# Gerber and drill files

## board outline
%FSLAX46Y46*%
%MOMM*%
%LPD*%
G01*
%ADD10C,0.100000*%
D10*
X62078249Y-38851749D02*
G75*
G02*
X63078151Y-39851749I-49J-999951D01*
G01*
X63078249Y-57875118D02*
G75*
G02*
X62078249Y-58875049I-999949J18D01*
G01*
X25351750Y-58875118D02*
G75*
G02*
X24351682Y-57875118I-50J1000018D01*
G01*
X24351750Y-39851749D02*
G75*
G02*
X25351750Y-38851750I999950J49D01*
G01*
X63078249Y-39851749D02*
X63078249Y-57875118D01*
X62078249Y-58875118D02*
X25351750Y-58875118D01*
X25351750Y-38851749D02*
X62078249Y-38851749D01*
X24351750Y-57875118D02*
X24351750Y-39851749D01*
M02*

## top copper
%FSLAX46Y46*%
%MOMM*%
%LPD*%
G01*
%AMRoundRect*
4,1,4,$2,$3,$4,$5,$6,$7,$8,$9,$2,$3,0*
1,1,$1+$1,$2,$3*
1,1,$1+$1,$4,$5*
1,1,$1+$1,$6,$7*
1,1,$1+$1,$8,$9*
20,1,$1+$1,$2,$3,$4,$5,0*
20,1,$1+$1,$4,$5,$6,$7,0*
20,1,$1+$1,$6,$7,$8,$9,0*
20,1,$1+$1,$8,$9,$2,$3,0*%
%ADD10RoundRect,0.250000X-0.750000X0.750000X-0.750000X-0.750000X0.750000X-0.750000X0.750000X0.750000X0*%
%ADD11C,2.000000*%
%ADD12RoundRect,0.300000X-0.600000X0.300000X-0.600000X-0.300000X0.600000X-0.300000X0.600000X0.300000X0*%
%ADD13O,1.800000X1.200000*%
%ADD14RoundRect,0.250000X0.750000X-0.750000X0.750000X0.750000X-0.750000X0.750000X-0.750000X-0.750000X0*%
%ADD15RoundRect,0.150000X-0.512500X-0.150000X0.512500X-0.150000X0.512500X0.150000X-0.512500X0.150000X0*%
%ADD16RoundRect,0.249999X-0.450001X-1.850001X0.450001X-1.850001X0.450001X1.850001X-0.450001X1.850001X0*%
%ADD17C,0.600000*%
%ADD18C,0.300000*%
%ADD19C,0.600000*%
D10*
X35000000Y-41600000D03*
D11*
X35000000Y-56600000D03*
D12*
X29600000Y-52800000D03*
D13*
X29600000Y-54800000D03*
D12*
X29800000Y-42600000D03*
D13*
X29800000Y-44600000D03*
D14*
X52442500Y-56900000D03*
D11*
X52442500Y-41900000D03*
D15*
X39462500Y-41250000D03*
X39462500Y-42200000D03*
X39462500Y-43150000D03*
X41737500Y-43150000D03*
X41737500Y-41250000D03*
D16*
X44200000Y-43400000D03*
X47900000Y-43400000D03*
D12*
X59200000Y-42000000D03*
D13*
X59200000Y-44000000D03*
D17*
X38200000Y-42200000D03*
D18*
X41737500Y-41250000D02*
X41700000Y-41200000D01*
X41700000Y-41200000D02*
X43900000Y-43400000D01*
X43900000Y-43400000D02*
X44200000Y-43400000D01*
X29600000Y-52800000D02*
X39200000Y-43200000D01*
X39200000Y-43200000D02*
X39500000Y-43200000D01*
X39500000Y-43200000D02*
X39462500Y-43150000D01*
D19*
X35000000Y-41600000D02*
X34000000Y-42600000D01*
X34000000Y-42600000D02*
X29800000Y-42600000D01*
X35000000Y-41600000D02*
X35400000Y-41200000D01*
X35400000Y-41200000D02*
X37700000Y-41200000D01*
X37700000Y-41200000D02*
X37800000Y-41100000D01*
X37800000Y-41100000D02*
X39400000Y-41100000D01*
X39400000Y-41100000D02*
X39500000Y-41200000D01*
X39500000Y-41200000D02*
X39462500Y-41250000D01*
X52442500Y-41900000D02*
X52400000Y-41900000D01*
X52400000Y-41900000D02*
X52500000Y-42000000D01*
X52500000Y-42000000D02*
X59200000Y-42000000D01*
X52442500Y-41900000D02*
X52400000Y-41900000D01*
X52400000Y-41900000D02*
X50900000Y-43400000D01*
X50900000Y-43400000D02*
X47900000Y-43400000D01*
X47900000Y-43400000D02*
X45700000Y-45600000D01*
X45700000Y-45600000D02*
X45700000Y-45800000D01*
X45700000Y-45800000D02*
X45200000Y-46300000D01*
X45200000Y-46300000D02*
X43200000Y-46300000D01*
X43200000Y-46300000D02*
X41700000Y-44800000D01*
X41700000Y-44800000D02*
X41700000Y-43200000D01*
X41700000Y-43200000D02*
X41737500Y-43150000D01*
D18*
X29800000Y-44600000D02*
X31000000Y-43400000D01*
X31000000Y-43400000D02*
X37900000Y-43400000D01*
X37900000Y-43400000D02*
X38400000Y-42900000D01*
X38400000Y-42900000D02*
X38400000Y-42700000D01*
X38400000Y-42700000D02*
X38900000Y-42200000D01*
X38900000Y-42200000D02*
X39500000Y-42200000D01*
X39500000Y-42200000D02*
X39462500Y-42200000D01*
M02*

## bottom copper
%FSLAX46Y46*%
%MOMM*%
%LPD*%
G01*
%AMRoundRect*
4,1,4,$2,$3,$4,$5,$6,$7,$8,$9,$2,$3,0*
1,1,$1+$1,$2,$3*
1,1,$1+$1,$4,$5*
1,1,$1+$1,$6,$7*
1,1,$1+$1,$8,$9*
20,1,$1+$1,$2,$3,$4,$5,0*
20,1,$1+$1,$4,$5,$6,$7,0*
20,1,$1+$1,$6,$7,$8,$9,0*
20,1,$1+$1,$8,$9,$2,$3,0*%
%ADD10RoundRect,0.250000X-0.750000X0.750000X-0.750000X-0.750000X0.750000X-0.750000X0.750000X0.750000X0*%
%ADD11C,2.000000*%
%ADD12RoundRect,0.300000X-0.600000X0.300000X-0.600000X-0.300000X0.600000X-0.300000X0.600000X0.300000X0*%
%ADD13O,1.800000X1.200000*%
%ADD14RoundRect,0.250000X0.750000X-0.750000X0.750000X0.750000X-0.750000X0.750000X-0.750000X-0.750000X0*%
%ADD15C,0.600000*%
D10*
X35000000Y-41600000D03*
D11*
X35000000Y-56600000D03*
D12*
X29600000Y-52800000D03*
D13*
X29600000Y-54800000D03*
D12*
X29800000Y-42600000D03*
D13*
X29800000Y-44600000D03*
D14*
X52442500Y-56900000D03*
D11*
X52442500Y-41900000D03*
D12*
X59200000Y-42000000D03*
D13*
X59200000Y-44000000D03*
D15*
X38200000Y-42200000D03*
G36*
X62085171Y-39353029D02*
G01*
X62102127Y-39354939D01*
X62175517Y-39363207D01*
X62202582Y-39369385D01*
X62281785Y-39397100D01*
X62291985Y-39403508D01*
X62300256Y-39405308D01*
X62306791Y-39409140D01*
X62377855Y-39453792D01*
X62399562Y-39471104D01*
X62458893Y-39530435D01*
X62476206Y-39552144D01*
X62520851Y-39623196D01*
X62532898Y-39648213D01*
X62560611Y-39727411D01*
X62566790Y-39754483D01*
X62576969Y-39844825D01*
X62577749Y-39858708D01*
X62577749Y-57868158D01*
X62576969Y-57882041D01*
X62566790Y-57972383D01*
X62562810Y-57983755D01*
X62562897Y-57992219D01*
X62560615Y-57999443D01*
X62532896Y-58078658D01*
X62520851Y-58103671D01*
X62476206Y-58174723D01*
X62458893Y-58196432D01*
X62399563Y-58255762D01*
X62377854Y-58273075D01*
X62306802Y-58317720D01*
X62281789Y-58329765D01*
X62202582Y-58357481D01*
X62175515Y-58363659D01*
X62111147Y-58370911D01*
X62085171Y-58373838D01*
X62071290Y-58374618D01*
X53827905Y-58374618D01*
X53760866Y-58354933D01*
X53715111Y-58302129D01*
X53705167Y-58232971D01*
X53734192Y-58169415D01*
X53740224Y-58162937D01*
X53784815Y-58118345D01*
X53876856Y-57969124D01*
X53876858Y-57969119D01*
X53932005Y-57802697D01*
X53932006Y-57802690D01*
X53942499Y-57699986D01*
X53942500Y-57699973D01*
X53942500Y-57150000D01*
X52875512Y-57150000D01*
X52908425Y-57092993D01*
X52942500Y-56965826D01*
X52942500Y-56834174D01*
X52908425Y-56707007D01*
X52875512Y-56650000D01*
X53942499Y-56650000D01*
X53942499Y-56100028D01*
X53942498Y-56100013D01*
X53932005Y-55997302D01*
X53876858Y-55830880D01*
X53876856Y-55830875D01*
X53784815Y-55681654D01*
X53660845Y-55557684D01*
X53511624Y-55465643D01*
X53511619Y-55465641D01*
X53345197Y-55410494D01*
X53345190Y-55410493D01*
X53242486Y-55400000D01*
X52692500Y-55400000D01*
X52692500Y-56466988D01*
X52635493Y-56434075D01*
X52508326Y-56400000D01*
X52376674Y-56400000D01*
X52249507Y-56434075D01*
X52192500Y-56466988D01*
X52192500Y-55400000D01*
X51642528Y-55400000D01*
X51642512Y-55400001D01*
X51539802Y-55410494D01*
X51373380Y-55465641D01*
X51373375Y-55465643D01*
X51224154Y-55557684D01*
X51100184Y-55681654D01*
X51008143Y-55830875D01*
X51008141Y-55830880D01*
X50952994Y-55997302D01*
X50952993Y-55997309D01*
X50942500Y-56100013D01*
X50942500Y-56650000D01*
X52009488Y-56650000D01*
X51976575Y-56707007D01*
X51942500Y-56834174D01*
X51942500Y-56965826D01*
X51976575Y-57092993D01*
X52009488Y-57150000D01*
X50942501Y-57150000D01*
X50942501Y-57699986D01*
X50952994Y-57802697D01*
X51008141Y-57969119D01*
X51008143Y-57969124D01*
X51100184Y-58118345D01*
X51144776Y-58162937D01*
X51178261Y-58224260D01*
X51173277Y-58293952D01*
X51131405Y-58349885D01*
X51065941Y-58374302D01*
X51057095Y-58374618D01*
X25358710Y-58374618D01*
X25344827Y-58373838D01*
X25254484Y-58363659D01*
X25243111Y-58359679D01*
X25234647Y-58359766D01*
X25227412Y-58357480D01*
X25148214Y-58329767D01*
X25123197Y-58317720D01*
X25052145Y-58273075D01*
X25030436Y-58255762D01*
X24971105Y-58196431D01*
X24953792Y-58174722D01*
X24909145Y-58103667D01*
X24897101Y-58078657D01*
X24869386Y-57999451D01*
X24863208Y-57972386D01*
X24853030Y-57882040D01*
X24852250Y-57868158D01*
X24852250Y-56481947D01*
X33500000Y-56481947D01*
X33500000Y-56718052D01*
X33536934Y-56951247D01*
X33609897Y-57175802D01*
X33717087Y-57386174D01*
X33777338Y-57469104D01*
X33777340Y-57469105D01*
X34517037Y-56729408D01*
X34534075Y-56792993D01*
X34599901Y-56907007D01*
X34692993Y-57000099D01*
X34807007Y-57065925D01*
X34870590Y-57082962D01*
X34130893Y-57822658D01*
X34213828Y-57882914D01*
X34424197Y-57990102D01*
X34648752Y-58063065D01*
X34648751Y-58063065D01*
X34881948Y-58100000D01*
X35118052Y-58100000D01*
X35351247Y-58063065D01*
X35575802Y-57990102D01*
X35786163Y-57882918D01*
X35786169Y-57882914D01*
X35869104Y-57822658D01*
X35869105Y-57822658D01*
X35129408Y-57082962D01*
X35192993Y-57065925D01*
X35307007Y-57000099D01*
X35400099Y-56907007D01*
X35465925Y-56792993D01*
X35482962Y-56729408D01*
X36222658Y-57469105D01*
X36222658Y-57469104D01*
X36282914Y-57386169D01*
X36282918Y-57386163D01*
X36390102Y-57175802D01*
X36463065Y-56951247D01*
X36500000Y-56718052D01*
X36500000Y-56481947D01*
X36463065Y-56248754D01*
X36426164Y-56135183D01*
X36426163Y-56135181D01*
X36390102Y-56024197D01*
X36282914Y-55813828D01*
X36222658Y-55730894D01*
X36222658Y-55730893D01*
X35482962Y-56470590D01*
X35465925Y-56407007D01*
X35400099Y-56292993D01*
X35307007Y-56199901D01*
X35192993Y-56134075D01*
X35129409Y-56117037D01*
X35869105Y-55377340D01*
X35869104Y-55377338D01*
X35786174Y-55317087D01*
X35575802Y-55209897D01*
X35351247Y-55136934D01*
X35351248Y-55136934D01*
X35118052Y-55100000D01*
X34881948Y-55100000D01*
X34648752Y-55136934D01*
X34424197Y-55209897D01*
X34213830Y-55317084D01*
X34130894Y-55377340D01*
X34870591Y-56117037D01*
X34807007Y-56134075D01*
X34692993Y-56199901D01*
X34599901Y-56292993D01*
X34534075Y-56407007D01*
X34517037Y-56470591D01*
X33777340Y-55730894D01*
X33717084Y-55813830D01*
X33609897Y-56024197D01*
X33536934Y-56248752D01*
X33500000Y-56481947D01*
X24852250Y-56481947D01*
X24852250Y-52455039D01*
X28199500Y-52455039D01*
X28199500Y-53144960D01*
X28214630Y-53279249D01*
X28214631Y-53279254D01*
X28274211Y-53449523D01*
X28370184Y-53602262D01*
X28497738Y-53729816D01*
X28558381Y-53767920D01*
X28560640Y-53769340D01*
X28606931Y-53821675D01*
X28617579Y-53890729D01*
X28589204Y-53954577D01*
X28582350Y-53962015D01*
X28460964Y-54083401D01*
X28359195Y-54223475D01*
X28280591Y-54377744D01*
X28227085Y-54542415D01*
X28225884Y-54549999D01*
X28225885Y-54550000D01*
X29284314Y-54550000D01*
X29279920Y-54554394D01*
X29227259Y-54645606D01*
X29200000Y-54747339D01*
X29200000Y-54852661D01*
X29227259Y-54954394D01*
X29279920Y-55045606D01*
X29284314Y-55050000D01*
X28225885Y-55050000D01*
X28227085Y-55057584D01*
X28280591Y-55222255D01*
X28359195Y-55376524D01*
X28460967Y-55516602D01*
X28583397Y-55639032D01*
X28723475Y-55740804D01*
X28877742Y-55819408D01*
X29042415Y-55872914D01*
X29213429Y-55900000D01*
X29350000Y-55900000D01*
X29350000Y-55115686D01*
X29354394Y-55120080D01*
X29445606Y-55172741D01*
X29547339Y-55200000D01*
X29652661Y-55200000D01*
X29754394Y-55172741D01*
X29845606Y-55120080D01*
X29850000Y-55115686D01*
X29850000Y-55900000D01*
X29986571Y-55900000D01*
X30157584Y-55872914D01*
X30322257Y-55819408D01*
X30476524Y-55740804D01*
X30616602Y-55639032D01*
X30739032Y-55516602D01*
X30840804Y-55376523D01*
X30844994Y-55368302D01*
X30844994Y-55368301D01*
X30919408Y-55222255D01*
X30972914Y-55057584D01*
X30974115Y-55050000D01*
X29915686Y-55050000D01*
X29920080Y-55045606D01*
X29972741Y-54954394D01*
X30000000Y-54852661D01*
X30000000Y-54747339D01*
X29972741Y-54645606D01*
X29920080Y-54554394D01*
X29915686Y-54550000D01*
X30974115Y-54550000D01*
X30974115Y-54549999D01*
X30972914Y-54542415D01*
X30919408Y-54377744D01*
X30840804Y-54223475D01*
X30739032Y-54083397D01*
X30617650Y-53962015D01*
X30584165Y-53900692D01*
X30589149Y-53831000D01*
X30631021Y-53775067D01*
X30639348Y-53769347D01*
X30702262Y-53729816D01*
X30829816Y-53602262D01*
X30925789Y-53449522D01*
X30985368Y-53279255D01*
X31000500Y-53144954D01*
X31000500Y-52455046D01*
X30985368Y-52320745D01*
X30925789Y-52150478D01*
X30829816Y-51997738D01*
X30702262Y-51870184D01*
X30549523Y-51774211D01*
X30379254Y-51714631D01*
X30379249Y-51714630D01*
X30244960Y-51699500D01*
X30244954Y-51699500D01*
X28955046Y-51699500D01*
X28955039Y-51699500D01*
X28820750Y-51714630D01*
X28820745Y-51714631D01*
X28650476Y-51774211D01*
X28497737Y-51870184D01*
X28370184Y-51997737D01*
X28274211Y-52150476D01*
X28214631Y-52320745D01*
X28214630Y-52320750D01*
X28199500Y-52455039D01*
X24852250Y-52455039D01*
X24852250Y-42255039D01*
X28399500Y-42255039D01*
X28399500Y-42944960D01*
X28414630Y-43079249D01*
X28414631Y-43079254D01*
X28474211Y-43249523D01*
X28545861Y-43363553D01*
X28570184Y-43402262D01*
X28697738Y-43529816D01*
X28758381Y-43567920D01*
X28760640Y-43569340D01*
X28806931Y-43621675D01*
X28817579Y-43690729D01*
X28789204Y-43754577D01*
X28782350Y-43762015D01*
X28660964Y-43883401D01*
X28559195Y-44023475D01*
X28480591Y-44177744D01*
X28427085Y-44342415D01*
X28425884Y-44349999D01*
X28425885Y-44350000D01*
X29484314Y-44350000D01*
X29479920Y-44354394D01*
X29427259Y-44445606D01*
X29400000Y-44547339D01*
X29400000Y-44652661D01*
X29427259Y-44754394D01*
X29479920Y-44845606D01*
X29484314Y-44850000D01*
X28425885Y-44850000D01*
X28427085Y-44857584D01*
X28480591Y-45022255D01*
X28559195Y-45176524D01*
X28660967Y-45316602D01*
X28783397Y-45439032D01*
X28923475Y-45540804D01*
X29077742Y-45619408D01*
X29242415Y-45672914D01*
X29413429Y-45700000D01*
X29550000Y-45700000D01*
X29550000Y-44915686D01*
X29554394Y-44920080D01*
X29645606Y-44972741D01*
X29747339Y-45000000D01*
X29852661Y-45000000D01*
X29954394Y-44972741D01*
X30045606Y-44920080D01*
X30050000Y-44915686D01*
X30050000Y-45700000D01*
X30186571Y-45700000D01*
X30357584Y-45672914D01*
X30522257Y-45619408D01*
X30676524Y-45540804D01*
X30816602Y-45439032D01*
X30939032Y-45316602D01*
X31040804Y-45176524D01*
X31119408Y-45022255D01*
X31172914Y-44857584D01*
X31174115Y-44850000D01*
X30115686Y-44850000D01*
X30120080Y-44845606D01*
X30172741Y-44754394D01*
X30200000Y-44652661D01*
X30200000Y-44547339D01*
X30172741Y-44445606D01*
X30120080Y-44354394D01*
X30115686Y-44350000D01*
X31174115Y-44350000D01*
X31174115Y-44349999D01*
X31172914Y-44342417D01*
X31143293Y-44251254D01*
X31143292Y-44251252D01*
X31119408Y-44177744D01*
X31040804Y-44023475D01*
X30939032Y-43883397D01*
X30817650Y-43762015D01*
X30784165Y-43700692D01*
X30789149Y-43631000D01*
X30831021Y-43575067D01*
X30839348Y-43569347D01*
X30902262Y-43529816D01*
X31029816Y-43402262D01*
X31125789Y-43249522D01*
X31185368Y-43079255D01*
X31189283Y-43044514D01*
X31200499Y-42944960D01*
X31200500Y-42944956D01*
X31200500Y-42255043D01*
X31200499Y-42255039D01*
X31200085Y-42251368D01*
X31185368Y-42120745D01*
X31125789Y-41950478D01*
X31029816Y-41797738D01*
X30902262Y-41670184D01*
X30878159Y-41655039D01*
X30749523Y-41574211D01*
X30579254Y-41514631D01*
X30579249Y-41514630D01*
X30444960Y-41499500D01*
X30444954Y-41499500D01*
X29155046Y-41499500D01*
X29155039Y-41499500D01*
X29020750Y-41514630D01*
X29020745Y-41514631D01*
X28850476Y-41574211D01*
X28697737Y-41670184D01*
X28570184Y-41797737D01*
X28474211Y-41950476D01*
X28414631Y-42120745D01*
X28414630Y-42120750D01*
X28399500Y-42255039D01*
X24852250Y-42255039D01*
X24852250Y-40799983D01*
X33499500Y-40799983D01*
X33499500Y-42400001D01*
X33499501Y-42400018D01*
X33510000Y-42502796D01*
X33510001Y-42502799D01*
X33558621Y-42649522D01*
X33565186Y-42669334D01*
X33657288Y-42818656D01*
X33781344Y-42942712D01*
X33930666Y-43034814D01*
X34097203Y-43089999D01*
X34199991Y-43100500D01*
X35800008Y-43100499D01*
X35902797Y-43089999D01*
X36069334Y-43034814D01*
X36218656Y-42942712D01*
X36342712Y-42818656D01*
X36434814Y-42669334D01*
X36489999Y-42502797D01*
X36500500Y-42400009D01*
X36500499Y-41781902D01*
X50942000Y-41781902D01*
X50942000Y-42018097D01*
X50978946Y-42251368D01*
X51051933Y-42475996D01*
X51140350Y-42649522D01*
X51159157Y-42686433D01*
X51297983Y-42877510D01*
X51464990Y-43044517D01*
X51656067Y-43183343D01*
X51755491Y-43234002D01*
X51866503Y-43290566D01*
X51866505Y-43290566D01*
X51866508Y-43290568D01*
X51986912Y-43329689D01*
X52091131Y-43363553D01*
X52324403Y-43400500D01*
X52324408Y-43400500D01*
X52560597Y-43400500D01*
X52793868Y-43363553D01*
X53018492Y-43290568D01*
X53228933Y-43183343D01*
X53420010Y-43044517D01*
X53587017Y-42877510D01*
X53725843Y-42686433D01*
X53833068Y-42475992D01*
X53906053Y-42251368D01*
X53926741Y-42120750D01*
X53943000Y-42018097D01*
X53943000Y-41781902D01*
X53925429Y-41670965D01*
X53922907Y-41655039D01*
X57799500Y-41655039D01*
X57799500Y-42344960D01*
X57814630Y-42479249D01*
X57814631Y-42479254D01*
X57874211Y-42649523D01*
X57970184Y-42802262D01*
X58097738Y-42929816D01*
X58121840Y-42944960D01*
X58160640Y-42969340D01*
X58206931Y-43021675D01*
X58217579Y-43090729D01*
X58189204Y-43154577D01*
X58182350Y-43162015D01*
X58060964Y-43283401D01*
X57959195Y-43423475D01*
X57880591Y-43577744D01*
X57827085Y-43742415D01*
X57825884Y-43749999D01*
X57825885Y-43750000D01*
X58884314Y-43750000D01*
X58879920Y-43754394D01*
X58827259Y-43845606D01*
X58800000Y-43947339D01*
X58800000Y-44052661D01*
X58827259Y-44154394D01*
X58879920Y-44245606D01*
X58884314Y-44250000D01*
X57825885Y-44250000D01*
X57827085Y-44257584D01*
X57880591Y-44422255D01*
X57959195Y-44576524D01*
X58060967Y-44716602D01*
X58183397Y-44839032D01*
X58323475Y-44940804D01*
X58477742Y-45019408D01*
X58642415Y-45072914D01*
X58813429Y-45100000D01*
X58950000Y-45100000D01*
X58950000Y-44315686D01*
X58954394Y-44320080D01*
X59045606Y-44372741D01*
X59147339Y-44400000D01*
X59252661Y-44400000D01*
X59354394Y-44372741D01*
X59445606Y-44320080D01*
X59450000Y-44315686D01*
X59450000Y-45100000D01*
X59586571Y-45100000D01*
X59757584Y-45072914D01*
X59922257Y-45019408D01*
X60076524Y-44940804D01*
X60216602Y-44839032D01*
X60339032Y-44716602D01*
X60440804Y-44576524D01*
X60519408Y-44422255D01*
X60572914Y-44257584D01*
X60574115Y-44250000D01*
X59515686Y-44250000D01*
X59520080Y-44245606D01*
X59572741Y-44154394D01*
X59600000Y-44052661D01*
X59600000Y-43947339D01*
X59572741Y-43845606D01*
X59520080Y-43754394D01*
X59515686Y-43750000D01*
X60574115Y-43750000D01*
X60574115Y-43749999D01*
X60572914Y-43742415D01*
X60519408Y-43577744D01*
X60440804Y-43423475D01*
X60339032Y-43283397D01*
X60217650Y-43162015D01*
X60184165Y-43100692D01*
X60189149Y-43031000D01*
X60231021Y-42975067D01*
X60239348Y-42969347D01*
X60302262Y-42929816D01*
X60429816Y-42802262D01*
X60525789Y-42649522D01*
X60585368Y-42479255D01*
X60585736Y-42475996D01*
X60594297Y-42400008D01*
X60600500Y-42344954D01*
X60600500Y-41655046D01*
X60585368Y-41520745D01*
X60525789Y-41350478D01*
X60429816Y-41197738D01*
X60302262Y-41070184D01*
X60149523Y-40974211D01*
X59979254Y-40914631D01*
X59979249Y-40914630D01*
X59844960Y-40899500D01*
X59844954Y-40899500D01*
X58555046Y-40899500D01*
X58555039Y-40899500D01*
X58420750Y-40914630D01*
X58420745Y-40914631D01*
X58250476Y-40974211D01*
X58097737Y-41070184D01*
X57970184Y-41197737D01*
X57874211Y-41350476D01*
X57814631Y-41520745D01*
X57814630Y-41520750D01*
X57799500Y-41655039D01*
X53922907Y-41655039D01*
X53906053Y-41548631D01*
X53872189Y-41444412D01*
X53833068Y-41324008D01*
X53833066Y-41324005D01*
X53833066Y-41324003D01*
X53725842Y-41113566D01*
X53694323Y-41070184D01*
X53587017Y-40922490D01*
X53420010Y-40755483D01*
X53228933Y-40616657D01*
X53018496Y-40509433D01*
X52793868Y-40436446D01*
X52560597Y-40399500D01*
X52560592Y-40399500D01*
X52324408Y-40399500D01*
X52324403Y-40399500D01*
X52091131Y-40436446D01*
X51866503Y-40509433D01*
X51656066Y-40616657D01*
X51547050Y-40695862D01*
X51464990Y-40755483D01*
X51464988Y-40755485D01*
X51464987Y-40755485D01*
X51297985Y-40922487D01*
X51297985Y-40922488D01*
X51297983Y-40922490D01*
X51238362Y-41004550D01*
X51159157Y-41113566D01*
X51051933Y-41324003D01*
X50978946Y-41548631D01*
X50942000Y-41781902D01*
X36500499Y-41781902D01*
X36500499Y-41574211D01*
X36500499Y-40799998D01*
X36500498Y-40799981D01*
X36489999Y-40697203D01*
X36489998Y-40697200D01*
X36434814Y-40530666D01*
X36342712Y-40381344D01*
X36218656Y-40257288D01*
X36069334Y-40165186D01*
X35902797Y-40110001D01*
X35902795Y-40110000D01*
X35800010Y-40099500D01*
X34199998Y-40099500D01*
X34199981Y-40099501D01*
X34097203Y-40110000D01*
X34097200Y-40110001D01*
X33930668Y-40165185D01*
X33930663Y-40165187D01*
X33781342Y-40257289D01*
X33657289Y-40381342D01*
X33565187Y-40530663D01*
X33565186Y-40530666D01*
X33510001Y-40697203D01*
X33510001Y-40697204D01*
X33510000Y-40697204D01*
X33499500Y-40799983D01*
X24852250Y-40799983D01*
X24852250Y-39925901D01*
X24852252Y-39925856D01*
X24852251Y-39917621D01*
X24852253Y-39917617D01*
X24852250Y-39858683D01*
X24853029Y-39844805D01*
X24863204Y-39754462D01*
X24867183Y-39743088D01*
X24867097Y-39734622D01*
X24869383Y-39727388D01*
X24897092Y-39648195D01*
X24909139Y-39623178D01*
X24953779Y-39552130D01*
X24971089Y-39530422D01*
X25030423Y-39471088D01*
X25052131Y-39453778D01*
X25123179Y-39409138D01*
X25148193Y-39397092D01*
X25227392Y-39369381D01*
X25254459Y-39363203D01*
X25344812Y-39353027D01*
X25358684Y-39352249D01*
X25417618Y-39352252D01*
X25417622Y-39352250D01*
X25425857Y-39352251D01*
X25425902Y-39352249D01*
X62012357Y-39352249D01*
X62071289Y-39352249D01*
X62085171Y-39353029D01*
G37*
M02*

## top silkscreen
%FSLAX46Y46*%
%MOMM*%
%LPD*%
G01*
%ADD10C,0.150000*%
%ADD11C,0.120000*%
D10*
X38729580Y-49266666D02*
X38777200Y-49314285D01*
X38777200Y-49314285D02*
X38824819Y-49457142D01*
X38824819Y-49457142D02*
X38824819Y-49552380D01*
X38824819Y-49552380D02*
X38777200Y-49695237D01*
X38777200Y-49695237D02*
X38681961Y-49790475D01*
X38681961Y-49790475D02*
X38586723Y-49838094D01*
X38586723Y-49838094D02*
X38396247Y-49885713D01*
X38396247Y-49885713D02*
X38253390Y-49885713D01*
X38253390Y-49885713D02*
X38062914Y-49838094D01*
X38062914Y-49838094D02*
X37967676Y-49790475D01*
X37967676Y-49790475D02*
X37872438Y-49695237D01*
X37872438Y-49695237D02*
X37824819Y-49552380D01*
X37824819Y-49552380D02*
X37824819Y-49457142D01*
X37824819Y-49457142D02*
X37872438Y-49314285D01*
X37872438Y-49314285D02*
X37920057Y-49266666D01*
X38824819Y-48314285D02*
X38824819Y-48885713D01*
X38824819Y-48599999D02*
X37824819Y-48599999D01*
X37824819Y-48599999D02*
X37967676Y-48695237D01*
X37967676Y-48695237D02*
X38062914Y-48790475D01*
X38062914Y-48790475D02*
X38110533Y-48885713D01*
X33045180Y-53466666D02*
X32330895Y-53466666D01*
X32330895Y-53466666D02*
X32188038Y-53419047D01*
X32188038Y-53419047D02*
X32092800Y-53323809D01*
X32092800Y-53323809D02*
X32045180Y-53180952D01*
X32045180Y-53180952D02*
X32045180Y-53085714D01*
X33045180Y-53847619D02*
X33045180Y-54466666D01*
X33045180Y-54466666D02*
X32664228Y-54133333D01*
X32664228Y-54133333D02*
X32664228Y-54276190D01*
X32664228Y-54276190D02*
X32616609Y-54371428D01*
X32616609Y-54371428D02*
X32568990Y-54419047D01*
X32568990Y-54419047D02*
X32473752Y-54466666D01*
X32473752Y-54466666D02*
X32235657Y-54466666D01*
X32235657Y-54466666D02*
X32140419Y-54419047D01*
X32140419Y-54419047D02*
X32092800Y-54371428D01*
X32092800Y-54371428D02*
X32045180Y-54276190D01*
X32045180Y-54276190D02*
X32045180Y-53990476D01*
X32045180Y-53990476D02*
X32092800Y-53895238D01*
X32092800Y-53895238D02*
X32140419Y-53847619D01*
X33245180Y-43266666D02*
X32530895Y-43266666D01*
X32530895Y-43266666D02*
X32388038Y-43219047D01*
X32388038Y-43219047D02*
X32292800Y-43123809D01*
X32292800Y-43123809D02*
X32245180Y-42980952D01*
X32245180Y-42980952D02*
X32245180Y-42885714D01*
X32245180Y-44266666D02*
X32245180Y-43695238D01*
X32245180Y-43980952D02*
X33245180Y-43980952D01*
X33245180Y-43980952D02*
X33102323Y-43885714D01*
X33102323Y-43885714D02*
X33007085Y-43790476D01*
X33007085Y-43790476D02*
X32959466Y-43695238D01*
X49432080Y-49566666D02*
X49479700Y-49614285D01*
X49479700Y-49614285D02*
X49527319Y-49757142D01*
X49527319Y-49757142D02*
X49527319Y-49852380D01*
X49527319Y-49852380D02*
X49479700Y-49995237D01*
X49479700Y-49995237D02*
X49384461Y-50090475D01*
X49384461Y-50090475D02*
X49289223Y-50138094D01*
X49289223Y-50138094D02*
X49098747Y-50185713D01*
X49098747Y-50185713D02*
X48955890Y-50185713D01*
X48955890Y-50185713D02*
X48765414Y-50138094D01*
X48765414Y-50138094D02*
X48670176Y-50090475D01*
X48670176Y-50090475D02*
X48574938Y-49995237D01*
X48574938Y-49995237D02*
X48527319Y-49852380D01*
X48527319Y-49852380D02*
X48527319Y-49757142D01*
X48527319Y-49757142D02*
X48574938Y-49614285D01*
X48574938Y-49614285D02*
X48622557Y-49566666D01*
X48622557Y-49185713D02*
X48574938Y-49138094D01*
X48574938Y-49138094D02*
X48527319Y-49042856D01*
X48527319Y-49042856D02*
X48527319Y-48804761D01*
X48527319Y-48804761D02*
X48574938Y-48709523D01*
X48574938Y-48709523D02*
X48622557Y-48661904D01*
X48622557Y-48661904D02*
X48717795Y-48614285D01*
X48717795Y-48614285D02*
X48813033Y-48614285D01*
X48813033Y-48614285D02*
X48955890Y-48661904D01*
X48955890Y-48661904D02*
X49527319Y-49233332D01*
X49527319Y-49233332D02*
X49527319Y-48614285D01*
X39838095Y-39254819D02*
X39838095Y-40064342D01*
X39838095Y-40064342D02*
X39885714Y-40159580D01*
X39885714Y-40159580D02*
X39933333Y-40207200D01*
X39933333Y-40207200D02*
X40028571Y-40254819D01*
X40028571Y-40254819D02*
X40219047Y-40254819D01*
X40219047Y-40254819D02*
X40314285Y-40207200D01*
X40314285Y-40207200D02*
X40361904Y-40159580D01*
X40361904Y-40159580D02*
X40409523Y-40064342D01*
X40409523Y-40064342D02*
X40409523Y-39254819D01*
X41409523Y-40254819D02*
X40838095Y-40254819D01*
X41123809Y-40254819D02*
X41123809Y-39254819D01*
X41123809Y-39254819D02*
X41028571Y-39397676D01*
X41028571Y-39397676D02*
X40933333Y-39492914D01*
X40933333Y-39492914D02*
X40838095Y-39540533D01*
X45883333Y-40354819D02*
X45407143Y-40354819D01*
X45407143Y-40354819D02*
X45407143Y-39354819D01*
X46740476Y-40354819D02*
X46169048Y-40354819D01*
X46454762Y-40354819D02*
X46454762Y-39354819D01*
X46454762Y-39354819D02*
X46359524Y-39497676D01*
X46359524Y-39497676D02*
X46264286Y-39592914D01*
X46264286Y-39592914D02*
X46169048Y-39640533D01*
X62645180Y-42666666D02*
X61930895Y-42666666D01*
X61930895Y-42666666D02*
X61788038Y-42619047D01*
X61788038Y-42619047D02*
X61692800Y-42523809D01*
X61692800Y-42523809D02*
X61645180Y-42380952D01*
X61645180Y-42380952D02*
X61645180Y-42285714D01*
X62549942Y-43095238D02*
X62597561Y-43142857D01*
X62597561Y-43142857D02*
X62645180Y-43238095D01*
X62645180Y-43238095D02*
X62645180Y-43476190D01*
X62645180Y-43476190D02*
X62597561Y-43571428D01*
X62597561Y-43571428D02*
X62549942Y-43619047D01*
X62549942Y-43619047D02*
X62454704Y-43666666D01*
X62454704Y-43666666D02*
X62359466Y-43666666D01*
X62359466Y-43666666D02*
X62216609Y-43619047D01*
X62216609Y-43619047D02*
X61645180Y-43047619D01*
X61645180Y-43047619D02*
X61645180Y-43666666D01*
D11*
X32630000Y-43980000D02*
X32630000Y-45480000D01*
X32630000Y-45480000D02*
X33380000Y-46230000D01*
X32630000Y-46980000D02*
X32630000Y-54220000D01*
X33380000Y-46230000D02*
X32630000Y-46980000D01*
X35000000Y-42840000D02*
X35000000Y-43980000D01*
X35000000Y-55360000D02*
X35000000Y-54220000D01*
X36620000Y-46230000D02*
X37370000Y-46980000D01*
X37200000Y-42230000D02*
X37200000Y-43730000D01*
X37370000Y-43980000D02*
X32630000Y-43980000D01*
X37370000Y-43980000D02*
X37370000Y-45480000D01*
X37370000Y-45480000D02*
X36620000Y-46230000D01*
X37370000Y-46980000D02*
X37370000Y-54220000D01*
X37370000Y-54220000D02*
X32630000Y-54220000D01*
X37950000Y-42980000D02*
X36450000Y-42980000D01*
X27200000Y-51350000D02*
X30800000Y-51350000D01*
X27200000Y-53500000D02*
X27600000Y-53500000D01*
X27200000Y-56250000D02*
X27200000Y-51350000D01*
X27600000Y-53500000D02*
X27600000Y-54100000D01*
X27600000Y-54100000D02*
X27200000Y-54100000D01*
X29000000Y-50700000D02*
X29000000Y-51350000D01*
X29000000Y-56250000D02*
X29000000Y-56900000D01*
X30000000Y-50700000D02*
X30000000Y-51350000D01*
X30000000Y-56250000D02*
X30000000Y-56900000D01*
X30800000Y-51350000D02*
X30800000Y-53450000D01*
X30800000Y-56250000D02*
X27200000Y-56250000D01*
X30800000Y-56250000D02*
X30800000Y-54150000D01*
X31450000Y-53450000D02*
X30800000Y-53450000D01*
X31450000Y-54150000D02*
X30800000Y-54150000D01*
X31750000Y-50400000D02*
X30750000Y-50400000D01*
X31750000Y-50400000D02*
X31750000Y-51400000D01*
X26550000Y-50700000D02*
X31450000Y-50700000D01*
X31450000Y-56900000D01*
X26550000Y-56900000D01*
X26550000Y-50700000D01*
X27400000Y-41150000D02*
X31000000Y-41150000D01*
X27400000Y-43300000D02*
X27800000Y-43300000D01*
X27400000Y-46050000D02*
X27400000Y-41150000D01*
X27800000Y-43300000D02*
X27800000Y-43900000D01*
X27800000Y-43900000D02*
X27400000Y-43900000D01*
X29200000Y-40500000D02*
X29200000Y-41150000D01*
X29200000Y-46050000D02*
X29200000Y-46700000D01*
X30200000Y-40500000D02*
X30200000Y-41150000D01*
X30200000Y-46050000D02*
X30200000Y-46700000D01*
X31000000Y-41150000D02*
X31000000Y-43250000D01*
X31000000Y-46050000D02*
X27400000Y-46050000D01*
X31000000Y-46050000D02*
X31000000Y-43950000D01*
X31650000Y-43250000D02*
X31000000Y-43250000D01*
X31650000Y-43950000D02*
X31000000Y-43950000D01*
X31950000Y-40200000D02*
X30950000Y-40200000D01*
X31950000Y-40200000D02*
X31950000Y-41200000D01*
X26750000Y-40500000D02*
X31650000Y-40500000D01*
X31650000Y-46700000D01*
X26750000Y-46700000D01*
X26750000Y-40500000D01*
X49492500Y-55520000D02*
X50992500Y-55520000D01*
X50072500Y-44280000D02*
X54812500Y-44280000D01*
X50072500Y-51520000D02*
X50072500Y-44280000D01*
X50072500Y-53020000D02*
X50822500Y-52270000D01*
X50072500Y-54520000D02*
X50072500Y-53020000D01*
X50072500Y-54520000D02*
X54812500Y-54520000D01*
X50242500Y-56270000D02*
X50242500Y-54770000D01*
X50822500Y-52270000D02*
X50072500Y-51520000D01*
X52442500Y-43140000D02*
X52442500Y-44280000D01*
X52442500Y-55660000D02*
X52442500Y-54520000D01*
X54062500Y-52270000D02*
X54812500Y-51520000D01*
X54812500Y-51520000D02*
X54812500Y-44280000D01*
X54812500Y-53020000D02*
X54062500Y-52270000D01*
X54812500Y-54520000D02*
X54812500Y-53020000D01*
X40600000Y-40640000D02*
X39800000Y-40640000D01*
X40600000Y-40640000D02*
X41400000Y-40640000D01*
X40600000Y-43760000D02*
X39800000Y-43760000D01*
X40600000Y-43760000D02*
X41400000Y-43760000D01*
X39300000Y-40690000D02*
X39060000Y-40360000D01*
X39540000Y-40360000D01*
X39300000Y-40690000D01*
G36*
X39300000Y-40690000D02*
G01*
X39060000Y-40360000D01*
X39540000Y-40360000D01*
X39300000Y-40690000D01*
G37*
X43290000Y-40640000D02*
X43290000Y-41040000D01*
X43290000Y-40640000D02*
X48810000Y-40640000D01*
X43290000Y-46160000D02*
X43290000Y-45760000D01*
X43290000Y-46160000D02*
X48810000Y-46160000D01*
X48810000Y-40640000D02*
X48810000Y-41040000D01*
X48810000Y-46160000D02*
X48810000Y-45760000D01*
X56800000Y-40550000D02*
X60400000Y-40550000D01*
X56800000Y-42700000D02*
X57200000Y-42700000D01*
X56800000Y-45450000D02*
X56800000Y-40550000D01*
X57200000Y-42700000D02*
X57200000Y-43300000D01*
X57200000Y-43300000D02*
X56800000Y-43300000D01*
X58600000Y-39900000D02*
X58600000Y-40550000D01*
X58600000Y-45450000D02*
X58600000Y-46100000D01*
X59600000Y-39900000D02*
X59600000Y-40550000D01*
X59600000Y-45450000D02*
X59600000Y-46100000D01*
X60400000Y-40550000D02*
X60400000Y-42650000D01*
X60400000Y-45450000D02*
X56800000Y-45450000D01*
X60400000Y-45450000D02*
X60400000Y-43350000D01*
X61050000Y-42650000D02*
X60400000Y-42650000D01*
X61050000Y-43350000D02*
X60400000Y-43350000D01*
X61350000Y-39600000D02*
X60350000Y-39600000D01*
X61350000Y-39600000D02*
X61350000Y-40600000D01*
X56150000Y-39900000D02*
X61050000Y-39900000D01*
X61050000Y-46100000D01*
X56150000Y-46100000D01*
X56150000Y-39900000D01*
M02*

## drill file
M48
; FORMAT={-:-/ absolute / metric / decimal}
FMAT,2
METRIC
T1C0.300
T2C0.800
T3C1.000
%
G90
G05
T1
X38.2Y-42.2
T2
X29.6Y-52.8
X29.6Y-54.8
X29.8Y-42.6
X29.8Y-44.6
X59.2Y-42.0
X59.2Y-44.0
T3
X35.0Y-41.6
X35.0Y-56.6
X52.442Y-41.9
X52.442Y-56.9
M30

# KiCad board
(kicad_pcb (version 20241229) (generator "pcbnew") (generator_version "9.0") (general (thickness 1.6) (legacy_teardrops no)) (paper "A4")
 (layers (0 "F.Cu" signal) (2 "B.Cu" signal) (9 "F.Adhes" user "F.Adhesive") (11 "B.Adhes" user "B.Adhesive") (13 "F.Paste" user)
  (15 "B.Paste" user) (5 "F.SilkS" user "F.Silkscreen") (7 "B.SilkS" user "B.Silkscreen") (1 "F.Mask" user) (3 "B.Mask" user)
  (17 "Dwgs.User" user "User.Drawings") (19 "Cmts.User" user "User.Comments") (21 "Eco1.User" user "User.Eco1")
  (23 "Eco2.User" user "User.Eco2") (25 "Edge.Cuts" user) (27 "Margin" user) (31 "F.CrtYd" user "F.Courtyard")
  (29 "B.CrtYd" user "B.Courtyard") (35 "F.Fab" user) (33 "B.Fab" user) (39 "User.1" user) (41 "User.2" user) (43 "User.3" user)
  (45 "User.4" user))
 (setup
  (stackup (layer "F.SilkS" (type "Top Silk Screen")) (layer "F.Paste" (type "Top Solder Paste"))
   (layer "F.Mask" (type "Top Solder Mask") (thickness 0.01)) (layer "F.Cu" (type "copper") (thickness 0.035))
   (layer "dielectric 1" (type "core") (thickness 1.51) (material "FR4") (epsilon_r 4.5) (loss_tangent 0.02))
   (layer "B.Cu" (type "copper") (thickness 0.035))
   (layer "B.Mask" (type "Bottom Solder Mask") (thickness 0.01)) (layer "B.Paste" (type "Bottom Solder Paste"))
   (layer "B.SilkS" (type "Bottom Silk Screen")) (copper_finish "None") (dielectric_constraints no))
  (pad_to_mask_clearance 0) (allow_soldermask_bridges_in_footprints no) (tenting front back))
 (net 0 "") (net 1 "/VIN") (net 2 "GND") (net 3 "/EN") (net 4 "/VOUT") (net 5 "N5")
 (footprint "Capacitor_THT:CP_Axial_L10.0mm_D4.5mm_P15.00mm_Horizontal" (layer "F.Cu") (at 35 41.6 -90)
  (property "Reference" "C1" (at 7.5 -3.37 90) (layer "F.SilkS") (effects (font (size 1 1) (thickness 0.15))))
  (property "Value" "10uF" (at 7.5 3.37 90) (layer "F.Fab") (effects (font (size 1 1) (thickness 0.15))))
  (fp_line (start 2.38 2.37) (end 3.88 2.37) (stroke (width 0.12) (type solid)) (layer "F.SilkS"))
  (fp_line (start 3.88 2.37) (end 4.63 1.62) (stroke (width 0.12) (type solid)) (layer "F.SilkS"))
  (fp_line (start 5.38 2.37) (end 12.62 2.37) (stroke (width 0.12) (type solid)) (layer "F.SilkS"))
  (fp_line (start 4.63 1.62) (end 5.38 2.37) (stroke (width 0.12) (type solid)) (layer "F.SilkS"))
  (fp_line (start 1.24 0) (end 2.38 0) (stroke (width 0.12) (type solid)) (layer "F.SilkS"))
  (fp_line (start 13.76 0) (end 12.62 0) (stroke (width 0.12) (type solid)) (layer "F.SilkS"))
  (fp_line (start 4.63 -1.62) (end 5.38 -2.37) (stroke (width 0.12) (type solid)) (layer "F.SilkS"))
  (fp_line (start 0.63 -2.2) (end 2.13 -2.2) (stroke (width 0.12) (type solid)) (layer "F.SilkS"))
  (fp_line (start 2.38 -2.37) (end 2.38 2.37) (stroke (width 0.12) (type solid)) (layer "F.SilkS"))
  (fp_line (start 2.38 -2.37) (end 3.88 -2.37) (stroke (width 0.12) (type solid)) (layer "F.SilkS"))
  (fp_line (start 3.88 -2.37) (end 4.63 -1.62) (stroke (width 0.12) (type solid)) (layer "F.SilkS"))
  (fp_line (start 5.38 -2.37) (end 12.62 -2.37) (stroke (width 0.12) (type solid)) (layer "F.SilkS"))
  (fp_line (start 12.62 -2.37) (end 12.62 2.37) (stroke (width 0.12) (type solid)) (layer "F.SilkS"))
  (fp_line (start 1.38 -2.95) (end 1.38 -1.45) (stroke (width 0.12) (type solid)) (layer "F.SilkS"))
  (pad "1" thru_hole roundrect (at 0 0 270) (size 2 2) (drill 1) (layers "*.Cu" "*.Mask") (remove_unused_layers no) (roundrect_rratio 0.125)
   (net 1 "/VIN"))
  (pad "2" thru_hole circle (at 15 0 270) (size 2 2) (drill 1) (layers "*.Cu" "*.Mask") (remove_unused_layers no) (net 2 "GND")))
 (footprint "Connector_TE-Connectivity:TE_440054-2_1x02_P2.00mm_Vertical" (layer "F.Cu") (at 29.6 52.8 -90)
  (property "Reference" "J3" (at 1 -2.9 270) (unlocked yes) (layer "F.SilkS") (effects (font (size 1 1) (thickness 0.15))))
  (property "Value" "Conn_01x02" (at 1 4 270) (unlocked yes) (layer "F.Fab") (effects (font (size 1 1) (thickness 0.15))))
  (fp_line (start -1.45 2.4) (end -1.45 -1.2) (stroke (width 0.12) (type solid)) (layer "F.SilkS"))
  (fp_line (start 0.7 2.4) (end 0.7 2) (stroke (width 0.12) (type solid)) (layer "F.SilkS"))
  (fp_line (start 3.45 2.4) (end -1.45 2.4) (stroke (width 0.12) (type solid)) (layer "F.SilkS"))
  (fp_line (start 0.7 2) (end 1.3 2) (stroke (width 0.12) (type solid)) (layer "F.SilkS"))
  (fp_line (start 1.3 2) (end 1.3 2.4) (stroke (width 0.12) (type solid)) (layer "F.SilkS"))
  (fp_line (start -2.1 0.6) (end -1.45 0.6) (stroke (width 0.12) (type solid)) (layer "F.SilkS"))
  (fp_line (start 3.45 0.6) (end 4.1 0.6) (stroke (width 0.12) (type solid)) (layer "F.SilkS"))
  (fp_line (start -2.1 -0.4) (end -1.45 -0.4) (stroke (width 0.12) (type solid)) (layer "F.SilkS"))
  (fp_line (start 3.45 -0.4) (end 4.1 -0.4) (stroke (width 0.12) (type solid)) (layer "F.SilkS"))
  (fp_line (start -1.45 -1.2) (end 0.65 -1.2) (stroke (width 0.12) (type solid)) (layer "F.SilkS"))
  (fp_line (start 3.45 -1.2) (end 3.45 2.4) (stroke (width 0.12) (type solid)) (layer "F.SilkS"))
  (fp_line (start 3.45 -1.2) (end 1.35 -1.2) (stroke (width 0.12) (type solid)) (layer "F.SilkS"))
  (fp_line (start 0.65 -1.85) (end 0.65 -1.2) (stroke (width 0.12) (type solid)) (layer "F.SilkS"))
  (fp_line (start 1.35 -1.85) (end 1.35 -1.2) (stroke (width 0.12) (type solid)) (layer "F.SilkS"))
  (fp_line (start -2.4 -2.15) (end -2.4 -1.15) (stroke (width 0.12) (type solid)) (layer "F.SilkS"))
  (fp_line (start -2.4 -2.15) (end -1.4 -2.15) (stroke (width 0.12) (type solid)) (layer "F.SilkS"))
  (fp_rect (start -2.1 -1.85) (end 4.1 3.05) (stroke (width 0.12) (type solid)) (fill no) (layer "F.SilkS"))
  (pad "1" thru_hole roundrect (at 0 0 270) (size 1.2 1.8) (drill 0.8) (layers "*.Cu" "*.Mask") (remove_unused_layers no)
   (roundrect_rratio 0.25) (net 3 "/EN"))
  (pad "2" thru_hole oval (at 2 0 270) (size 1.2 1.8) (drill 0.8) (layers "*.Cu" "*.Mask") (remove_unused_layers no) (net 2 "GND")))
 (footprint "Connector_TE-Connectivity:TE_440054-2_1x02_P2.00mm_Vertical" (layer "F.Cu") (at 29.8 42.6 -90)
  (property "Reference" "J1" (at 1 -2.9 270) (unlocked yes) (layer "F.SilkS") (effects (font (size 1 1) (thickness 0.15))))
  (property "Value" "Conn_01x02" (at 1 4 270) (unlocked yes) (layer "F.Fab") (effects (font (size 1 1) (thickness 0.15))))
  (fp_line (start -1.45 2.4) (end -1.45 -1.2) (stroke (width 0.12) (type solid)) (layer "F.SilkS"))
  (fp_line (start 0.7 2.4) (end 0.7 2) (stroke (width 0.12) (type solid)) (layer "F.SilkS"))
  (fp_line (start 3.45 2.4) (end -1.45 2.4) (stroke (width 0.12) (type solid)) (layer "F.SilkS"))
  (fp_line (start 0.7 2) (end 1.3 2) (stroke (width 0.12) (type solid)) (layer "F.SilkS"))
  (fp_line (start 1.3 2) (end 1.3 2.4) (stroke (width 0.12) (type solid)) (layer "F.SilkS"))
  (fp_line (start -2.1 0.6) (end -1.45 0.6) (stroke (width 0.12) (type solid)) (layer "F.SilkS"))
  (fp_line (start 3.45 0.6) (end 4.1 0.6) (stroke (width 0.12) (type solid)) (layer "F.SilkS"))
  (fp_line (start -2.1 -0.4) (end -1.45 -0.4) (stroke (width 0.12) (type solid)) (layer "F.SilkS"))
  (fp_line (start 3.45 -0.4) (end 4.1 -0.4) (stroke (width 0.12) (type solid)) (layer "F.SilkS"))
  (fp_line (start -1.45 -1.2) (end 0.65 -1.2) (stroke (width 0.12) (type solid)) (layer "F.SilkS"))
  (fp_line (start 3.45 -1.2) (end 3.45 2.4) (stroke (width 0.12) (type solid)) (layer "F.SilkS"))
  (fp_line (start 3.45 -1.2) (end 1.35 -1.2) (stroke (width 0.12) (type solid)) (layer "F.SilkS"))
  (fp_line (start 0.65 -1.85) (end 0.65 -1.2) (stroke (width 0.12) (type solid)) (layer "F.SilkS"))
  (fp_line (start 1.35 -1.85) (end 1.35 -1.2) (stroke (width 0.12) (type solid)) (layer "F.SilkS"))
  (fp_line (start -2.4 -2.15) (end -2.4 -1.15) (stroke (width 0.12) (type solid)) (layer "F.SilkS"))
  (fp_line (start -2.4 -2.15) (end -1.4 -2.15) (stroke (width 0.12) (type solid)) (layer "F.SilkS"))
  (fp_rect (start -2.1 -1.85) (end 4.1 3.05) (stroke (width 0.12) (type solid)) (fill no) (layer "F.SilkS"))
  (pad "1" thru_hole roundrect (at 0 0 270) (size 1.2 1.8) (drill 0.8) (layers "*.Cu" "*.Mask") (remove_unused_layers no)
   (roundrect_rratio 0.25) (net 1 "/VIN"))
  (pad "2" thru_hole oval (at 2 0 270) (size 1.2 1.8) (drill 0.8) (layers "*.Cu" "*.Mask") (remove_unused_layers no) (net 2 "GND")))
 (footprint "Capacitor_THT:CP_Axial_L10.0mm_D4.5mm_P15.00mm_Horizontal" (layer "F.Cu") (at 52.4425 56.9 90)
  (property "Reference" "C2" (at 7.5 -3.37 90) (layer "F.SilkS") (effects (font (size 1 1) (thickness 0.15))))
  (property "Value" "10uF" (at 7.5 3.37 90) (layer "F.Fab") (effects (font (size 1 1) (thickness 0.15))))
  (fp_line (start 1.38 -2.95) (end 1.38 -1.45) (stroke (width 0.12) (type solid)) (layer "F.SilkS"))
  (fp_line (start 12.62 -2.37) (end 12.62 2.37) (stroke (width 0.12) (type solid)) (layer "F.SilkS"))
  (fp_line (start 5.38 -2.37) (end 12.62 -2.37) (stroke (width 0.12) (type solid)) (layer "F.SilkS"))
  (fp_line (start 3.88 -2.37) (end 4.63 -1.62) (stroke (width 0.12) (type solid)) (layer "F.SilkS"))
  (fp_line (start 2.38 -2.37) (end 3.88 -2.37) (stroke (width 0.12) (type solid)) (layer "F.SilkS"))
  (fp_line (start 2.38 -2.37) (end 2.38 2.37) (stroke (width 0.12) (type solid)) (layer "F.SilkS"))
  (fp_line (start 0.63 -2.2) (end 2.13 -2.2) (stroke (width 0.12) (type solid)) (layer "F.SilkS"))
  (fp_line (start 4.63 -1.62) (end 5.38 -2.37) (stroke (width 0.12) (type solid)) (layer "F.SilkS"))
  (fp_line (start 13.76 0) (end 12.62 0) (stroke (width 0.12) (type solid)) (layer "F.SilkS"))
  (fp_line (start 1.24 0) (end 2.38 0) (stroke (width 0.12) (type solid)) (layer "F.SilkS"))
  (fp_line (start 4.63 1.62) (end 5.38 2.37) (stroke (width 0.12) (type solid)) (layer "F.SilkS"))
  (fp_line (start 5.38 2.37) (end 12.62 2.37) (stroke (width 0.12) (type solid)) (layer "F.SilkS"))
  (fp_line (start 3.88 2.37) (end 4.63 1.62) (stroke (width 0.12) (type solid)) (layer "F.SilkS"))
  (fp_line (start 2.38 2.37) (end 3.88 2.37) (stroke (width 0.12) (type solid)) (layer "F.SilkS"))
  (pad "1" thru_hole roundrect (at 0 0 90) (size 2 2) (drill 1) (layers "*.Cu" "*.Mask") (remove_unused_layers no) (roundrect_rratio 0.125)
   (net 2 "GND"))
  (pad "2" thru_hole circle (at 15 0 90) (size 2 2) (drill 1) (layers "*.Cu" "*.Mask") (remove_unused_layers no) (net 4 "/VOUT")))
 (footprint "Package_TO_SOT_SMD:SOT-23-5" (layer "F.Cu") (at 40.6 42.2)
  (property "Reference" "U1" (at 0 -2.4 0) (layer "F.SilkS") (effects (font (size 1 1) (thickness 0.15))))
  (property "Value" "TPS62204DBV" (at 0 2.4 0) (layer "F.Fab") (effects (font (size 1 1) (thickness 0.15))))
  (fp_line (start 0 -1.56) (end -0.8 -1.56) (stroke (width 0.12) (type solid)) (layer "F.SilkS"))
  (fp_line (start 0 -1.56) (end 0.8 -1.56) (stroke (width 0.12) (type solid)) (layer "F.SilkS"))
  (fp_line (start 0 1.56) (end -0.8 1.56) (stroke (width 0.12) (type solid)) (layer "F.SilkS"))
  (fp_line (start 0 1.56) (end 0.8 1.56) (stroke (width 0.12) (type solid)) (layer "F.SilkS"))
  (fp_poly (pts (xy -1.3 -1.51) (xy -1.54 -1.84) (xy -1.06 -1.84)) (stroke (width 0.12) (type solid)) (fill yes) (layer "F.SilkS"))
  (pad "1" smd roundrect (at -1.1375 -0.95) (size 1.325 0.6) (layers "F.Cu" "F.Mask" "F.Paste") (roundrect_rratio 0.25) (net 1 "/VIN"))
  (pad "2" smd roundrect (at -1.1375 0) (size 1.325 0.6) (layers "F.Cu" "F.Mask" "F.Paste") (roundrect_rratio 0.25) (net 2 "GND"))
  (pad "3" smd roundrect (at -1.1375 0.95) (size 1.325 0.6) (layers "F.Cu" "F.Mask" "F.Paste") (roundrect_rratio 0.25) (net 3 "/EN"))
  (pad "4" smd roundrect (at 1.1375 0.95) (size 1.325 0.6) (layers "F.Cu" "F.Mask" "F.Paste") (roundrect_rratio 0.25) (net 4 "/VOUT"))
  (pad "5" smd roundrect (at 1.1375 -0.95) (size 1.325 0.6) (layers "F.Cu" "F.Mask" "F.Paste") (roundrect_rratio 0.25) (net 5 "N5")))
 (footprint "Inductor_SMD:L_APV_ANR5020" (layer "F.Cu") (at 46.05 43.4)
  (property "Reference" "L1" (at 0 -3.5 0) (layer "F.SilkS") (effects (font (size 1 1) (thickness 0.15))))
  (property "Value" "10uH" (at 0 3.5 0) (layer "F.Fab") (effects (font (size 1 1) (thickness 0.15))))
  (fp_line (start -2.76 -2.76) (end -2.76 -2.36) (stroke (width 0.12) (type solid)) (layer "F.SilkS"))
  (fp_line (start -2.76 -2.76) (end 2.76 -2.76) (stroke (width 0.12) (type solid)) (layer "F.SilkS"))
  (fp_line (start -2.76 2.76) (end -2.76 2.36) (stroke (width 0.12) (type solid)) (layer "F.SilkS"))
  (fp_line (start -2.76 2.76) (end 2.76 2.76) (stroke (width 0.12) (type solid)) (layer "F.SilkS"))
  (fp_line (start 2.76 -2.76) (end 2.76 -2.36) (stroke (width 0.12) (type solid)) (layer "F.SilkS"))
  (fp_line (start 2.76 2.76) (end 2.76 2.36) (stroke (width 0.12) (type solid)) (layer "F.SilkS"))
  (pad "1" smd roundrect (at -1.85 0) (size 1.4 4.2) (layers "F.Cu" "F.Mask" "F.Paste") (roundrect_rratio 0.178571) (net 5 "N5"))
  (pad "2" smd roundrect (at 1.85 0) (size 1.4 4.2) (layers "F.Cu" "F.Mask" "F.Paste") (roundrect_rratio 0.178571) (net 4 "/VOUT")))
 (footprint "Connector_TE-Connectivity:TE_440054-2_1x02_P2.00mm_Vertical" (layer "F.Cu") (at 59.2 42 -90)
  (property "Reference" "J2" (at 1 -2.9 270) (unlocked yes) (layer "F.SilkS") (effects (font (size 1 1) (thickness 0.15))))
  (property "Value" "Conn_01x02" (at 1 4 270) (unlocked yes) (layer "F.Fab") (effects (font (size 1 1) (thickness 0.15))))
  (fp_line (start -1.45 2.4) (end -1.45 -1.2) (stroke (width 0.12) (type solid)) (layer "F.SilkS"))
  (fp_line (start 0.7 2.4) (end 0.7 2) (stroke (width 0.12) (type solid)) (layer "F.SilkS"))
  (fp_line (start 3.45 2.4) (end -1.45 2.4) (stroke (width 0.12) (type solid)) (layer "F.SilkS"))
  (fp_line (start 0.7 2) (end 1.3 2) (stroke (width 0.12) (type solid)) (layer "F.SilkS"))
  (fp_line (start 1.3 2) (end 1.3 2.4) (stroke (width 0.12) (type solid)) (layer "F.SilkS"))
  (fp_line (start -2.1 0.6) (end -1.45 0.6) (stroke (width 0.12) (type solid)) (layer "F.SilkS"))
  (fp_line (start 3.45 0.6) (end 4.1 0.6) (stroke (width 0.12) (type solid)) (layer "F.SilkS"))
  (fp_line (start -2.1 -0.4) (end -1.45 -0.4) (stroke (width 0.12) (type solid)) (layer "F.SilkS"))
  (fp_line (start 3.45 -0.4) (end 4.1 -0.4) (stroke (width 0.12) (type solid)) (layer "F.SilkS"))
  (fp_line (start -1.45 -1.2) (end 0.65 -1.2) (stroke (width 0.12) (type solid)) (layer "F.SilkS"))
  (fp_line (start 3.45 -1.2) (end 3.45 2.4) (stroke (width 0.12) (type solid)) (layer "F.SilkS"))
  (fp_line (start 3.45 -1.2) (end 1.35 -1.2) (stroke (width 0.12) (type solid)) (layer "F.SilkS"))
  (fp_line (start 0.65 -1.85) (end 0.65 -1.2) (stroke (width 0.12) (type solid)) (layer "F.SilkS"))
  (fp_line (start 1.35 -1.85) (end 1.35 -1.2) (stroke (width 0.12) (type solid)) (layer "F.SilkS"))
  (fp_line (start -2.4 -2.15) (end -2.4 -1.15) (stroke (width 0.12) (type solid)) (layer "F.SilkS"))
  (fp_line (start -2.4 -2.15) (end -1.4 -2.15) (stroke (width 0.12) (type solid)) (layer "F.SilkS"))
  (fp_rect (start -2.1 -1.85) (end 4.1 3.05) (stroke (width 0.12) (type solid)) (fill no) (layer "F.SilkS"))
  (pad "1" thru_hole roundrect (at 0 0 270) (size 1.2 1.8) (drill 0.8) (layers "*.Cu" "*.Mask") (remove_unused_layers no)
   (roundrect_rratio 0.25) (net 4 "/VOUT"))
  (pad "2" thru_hole oval (at 2 0 270) (size 1.2 1.8) (drill 0.8) (layers "*.Cu" "*.Mask") (remove_unused_layers no) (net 2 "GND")))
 (gr_arc (start 62.078249 38.851749) (mid 62.785356 39.144642) (end 63.078249 39.851749) (stroke (width 0.1) (type default))
  (layer "Edge.Cuts"))
 (gr_arc (start 63.078249 57.875118) (mid 62.785352 58.58223) (end 62.078249 58.875118) (stroke (width 0.1) (type default))
  (layer "Edge.Cuts"))
 (gr_arc (start 25.35175 58.875118) (mid 24.644643 58.582225) (end 24.35175 57.875118) (stroke (width 0.1) (type default))
  (layer "Edge.Cuts"))
 (gr_arc (start 24.35175 39.851749) (mid 24.644629 39.144628) (end 25.35175 38.851749) (stroke (width 0.1) (type default))
  (layer "Edge.Cuts"))
 (gr_line (start 63.078249 39.851749) (end 63.078249 57.875118) (stroke (width 0.1) (type default)) (layer "Edge.Cuts"))
 (gr_line (start 62.078249 58.875118) (end 25.35175 58.875118) (stroke (width 0.1) (type default)) (layer "Edge.Cuts"))
 (gr_line (start 25.35175 38.851749) (end 62.078249 38.851749) (stroke (width 0.1) (type default)) (layer "Edge.Cuts"))
 (gr_line (start 24.35175 57.875118) (end 24.35175 39.851749) (stroke (width 0.1) (type default)) (layer "Edge.Cuts"))
 (via (at 38.2 42.2) (size 0.6) (drill 0.3) (layers "F.Cu" "B.Cu") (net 2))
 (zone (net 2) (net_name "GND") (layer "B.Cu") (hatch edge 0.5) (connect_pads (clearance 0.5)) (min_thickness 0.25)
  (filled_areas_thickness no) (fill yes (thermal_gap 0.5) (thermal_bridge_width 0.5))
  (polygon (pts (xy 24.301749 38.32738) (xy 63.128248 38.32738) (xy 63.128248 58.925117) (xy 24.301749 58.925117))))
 (segment (start 41.737500 41.250000) (end 41.700000 41.200000) (width 0.3) (layer "F.Cu") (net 5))
 (segment (start 41.700000 41.200000) (end 43.900000 43.400000) (width 0.3) (layer "F.Cu") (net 5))
 (segment (start 43.900000 43.400000) (end 44.200000 43.400000) (width 0.3) (layer "F.Cu") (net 5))
 (segment (start 29.600000 52.800000) (end 39.200000 43.200000) (width 0.3) (layer "F.Cu") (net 3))
 (segment (start 39.200000 43.200000) (end 39.500000 43.200000) (width 0.3) (layer "F.Cu") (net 3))
 (segment (start 39.500000 43.200000) (end 39.462500 43.150000) (width 0.3) (layer "F.Cu") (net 3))
 (segment (start 35.000000 41.600000) (end 34.000000 42.600000) (width 0.6) (layer "F.Cu") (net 1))
 (segment (start 34.000000 42.600000) (end 29.800000 42.600000) (width 0.6) (layer "F.Cu") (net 1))
 (segment (start 35.000000 41.600000) (end 35.400000 41.200000) (width 0.6) (layer "F.Cu") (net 1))
 (segment (start 35.400000 41.200000) (end 37.700000 41.200000) (width 0.6) (layer "F.Cu") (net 1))
 (segment (start 37.700000 41.200000) (end 37.800000 41.100000) (width 0.6) (layer "F.Cu") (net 1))
 (segment (start 37.800000 41.100000) (end 39.400000 41.100000) (width 0.6) (layer "F.Cu") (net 1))
 (segment (start 39.400000 41.100000) (end 39.500000 41.200000) (width 0.6) (layer "F.Cu") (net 1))
 (segment (start 39.500000 41.200000) (end 39.462500 41.250000) (width 0.6) (layer "F.Cu") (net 1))
 (segment (start 52.442500 41.900000) (end 52.400000 41.900000) (width 0.6) (layer "F.Cu") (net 4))
 (segment (start 52.400000 41.900000) (end 52.500000 42.000000) (width 0.6) (layer "F.Cu") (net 4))
 (segment (start 52.500000 42.000000) (end 59.200000 42.000000) (width 0.6) (layer "F.Cu") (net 4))
 (segment (start 52.442500 41.900000) (end 52.400000 41.900000) (width 0.6) (layer "F.Cu") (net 4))
 (segment (start 52.400000 41.900000) (end 50.900000 43.400000) (width 0.6) (layer "F.Cu") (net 4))
 (segment (start 50.900000 43.400000) (end 47.900000 43.400000) (width 0.6) (layer "F.Cu") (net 4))
 (segment (start 47.900000 43.400000) (end 45.700000 45.600000) (width 0.6) (layer "F.Cu") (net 4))
 (segment (start 45.700000 45.600000) (end 45.700000 45.800000) (width 0.6) (layer "F.Cu") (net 4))
 (segment (start 45.700000 45.800000) (end 45.200000 46.300000) (width 0.6) (layer "F.Cu") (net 4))
 (segment (start 45.200000 46.300000) (end 43.200000 46.300000) (width 0.6) (layer "F.Cu") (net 4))
 (segment (start 43.200000 46.300000) (end 41.700000 44.800000) (width 0.6) (layer "F.Cu") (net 4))
 (segment (start 41.700000 44.800000) (end 41.700000 43.200000) (width 0.6) (layer "F.Cu") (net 4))
 (segment (start 41.700000 43.200000) (end 41.737500 43.150000) (width 0.6) (layer "F.Cu") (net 4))
 (segment (start 29.800000 44.600000) (end 31.000000 43.400000) (width 0.3) (layer "F.Cu") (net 2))
 (segment (start 31.000000 43.400000) (end 37.900000 43.400000) (width 0.3) (layer "F.Cu") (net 2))
 (segment (start 37.900000 43.400000) (end 38.400000 42.900000) (width 0.3) (layer "F.Cu") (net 2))
 (segment (start 38.400000 42.900000) (end 38.400000 42.700000) (width 0.3) (layer "F.Cu") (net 2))
 (segment (start 38.400000 42.700000) (end 38.900000 42.200000) (width 0.3) (layer "F.Cu") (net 2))
 (segment (start 38.900000 42.200000) (end 39.500000 42.200000) (width 0.3) (layer "F.Cu") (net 2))
 (segment (start 39.500000 42.200000) (end 39.462500 42.200000) (width 0.3) (layer "F.Cu") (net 2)))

